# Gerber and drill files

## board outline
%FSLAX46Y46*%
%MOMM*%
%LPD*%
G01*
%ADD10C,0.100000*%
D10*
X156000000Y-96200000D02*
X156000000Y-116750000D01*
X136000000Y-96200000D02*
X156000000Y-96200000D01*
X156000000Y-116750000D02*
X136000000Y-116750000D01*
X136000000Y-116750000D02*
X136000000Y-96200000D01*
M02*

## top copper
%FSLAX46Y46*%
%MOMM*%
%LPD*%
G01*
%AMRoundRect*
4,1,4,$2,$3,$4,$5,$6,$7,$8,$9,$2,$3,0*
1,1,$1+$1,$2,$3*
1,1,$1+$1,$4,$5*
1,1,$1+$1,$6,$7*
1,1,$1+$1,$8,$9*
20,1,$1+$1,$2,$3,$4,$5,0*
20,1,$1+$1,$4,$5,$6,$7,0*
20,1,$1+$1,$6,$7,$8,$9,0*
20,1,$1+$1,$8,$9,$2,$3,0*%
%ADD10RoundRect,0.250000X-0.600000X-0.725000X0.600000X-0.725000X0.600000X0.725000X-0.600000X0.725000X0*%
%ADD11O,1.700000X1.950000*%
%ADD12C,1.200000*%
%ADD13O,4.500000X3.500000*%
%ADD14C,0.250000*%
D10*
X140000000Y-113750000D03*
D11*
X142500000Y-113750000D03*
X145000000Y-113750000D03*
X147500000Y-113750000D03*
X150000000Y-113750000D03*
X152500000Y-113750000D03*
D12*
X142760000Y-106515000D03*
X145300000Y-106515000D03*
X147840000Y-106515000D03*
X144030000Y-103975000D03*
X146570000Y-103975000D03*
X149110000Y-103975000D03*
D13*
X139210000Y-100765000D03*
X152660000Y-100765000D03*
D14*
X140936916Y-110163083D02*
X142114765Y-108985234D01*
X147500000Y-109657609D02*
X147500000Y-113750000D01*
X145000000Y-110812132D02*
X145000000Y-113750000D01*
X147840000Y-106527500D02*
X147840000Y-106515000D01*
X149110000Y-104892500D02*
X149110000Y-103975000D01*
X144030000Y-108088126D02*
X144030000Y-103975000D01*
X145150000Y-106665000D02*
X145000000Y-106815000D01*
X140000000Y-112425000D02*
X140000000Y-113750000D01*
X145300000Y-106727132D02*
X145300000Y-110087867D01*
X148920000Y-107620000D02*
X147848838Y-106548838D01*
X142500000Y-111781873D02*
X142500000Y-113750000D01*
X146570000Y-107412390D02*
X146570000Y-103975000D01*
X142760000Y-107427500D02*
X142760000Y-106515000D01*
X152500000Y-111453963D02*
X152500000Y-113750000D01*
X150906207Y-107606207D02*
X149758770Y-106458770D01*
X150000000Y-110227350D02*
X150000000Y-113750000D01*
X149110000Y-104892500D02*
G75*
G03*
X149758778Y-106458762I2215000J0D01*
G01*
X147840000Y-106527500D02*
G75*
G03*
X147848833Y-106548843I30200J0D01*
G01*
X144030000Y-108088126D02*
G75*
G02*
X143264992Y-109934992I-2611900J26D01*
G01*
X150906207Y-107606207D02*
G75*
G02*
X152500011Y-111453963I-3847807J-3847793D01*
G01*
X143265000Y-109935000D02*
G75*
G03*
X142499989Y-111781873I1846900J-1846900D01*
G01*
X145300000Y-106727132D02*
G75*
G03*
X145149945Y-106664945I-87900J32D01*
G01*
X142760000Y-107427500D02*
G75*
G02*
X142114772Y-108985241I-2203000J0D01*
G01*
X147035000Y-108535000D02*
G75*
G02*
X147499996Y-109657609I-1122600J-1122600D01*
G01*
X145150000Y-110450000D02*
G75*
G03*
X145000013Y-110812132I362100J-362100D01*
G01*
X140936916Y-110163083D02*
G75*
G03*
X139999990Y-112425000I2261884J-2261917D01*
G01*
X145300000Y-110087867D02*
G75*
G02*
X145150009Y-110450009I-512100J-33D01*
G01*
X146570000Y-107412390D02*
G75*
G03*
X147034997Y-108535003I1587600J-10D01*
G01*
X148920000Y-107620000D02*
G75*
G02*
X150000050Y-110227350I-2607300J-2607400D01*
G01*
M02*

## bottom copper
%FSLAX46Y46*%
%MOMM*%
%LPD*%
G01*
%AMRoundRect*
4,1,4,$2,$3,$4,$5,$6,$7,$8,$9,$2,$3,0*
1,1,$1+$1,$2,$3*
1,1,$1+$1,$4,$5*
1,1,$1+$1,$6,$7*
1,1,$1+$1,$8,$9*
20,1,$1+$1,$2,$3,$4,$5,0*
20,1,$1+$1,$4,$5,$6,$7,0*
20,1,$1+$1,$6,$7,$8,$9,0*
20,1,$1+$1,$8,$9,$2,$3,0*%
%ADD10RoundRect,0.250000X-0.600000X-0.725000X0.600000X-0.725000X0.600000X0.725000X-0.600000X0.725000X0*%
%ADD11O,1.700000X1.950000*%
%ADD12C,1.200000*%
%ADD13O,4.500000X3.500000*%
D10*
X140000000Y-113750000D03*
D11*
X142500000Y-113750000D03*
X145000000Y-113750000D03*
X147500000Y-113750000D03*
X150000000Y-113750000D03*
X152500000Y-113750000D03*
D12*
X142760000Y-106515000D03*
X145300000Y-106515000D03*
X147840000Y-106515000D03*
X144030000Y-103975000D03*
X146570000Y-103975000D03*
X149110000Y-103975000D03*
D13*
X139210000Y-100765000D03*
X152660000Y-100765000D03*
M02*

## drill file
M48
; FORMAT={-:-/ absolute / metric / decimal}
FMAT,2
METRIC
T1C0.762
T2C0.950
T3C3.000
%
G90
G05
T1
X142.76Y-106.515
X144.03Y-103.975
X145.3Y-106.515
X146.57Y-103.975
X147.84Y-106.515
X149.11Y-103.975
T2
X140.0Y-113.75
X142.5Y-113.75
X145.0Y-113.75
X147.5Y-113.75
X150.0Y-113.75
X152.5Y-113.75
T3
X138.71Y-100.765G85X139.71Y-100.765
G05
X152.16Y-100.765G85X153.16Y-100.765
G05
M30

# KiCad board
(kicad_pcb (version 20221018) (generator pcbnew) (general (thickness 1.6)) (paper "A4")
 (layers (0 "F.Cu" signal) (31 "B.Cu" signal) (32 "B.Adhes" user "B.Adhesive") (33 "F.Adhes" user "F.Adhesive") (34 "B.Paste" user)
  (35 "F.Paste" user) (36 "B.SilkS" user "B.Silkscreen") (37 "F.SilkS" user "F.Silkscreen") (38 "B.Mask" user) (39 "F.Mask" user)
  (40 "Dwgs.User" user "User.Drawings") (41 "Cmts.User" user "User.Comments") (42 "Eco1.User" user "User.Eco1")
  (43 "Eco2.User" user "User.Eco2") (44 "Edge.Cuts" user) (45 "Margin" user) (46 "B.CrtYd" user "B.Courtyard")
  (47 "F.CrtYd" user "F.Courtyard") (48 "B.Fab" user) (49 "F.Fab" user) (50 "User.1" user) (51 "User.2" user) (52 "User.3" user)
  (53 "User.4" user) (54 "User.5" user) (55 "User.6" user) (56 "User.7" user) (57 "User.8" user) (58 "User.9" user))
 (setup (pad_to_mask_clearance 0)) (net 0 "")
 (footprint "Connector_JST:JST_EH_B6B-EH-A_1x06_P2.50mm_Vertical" (layer "F.Cu") (at 140 113.75)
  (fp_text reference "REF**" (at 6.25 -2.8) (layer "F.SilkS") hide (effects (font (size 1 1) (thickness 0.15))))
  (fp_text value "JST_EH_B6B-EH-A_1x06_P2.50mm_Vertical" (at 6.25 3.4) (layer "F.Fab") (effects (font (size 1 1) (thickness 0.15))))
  (pad "1" thru_hole roundrect (at 0 0) (size 1.7 1.95) (drill 0.95) (layers "*.Cu" "*.Mask") (roundrect_rratio 0.1470588235))
  (pad "2" thru_hole oval (at 2.5 0) (size 1.7 1.95) (drill 0.95) (layers "*.Cu" "*.Mask"))
  (pad "3" thru_hole oval (at 5 0) (size 1.7 1.95) (drill 0.95) (layers "*.Cu" "*.Mask"))
  (pad "4" thru_hole oval (at 7.5 0) (size 1.7 1.95) (drill 0.95) (layers "*.Cu" "*.Mask"))
  (pad "5" thru_hole oval (at 10 0) (size 1.7 1.95) (drill 0.95) (layers "*.Cu" "*.Mask"))
  (pad "6" thru_hole oval (at 12.5 0) (size 1.7 1.95) (drill 0.95) (layers "*.Cu" "*.Mask")))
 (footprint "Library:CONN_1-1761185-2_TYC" (layer "F.Cu") (at 142.76 106.515)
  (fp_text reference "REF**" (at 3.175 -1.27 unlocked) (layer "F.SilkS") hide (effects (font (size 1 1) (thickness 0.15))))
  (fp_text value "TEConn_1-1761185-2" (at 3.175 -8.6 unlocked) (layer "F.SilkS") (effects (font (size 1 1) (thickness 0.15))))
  (pad "1" thru_hole circle (at 0 0) (size 1.2 1.2) (drill 0.762) (layers "*.Cu" "*.Mask"))
  (pad "3" thru_hole circle (at 2.54 0) (size 1.2 1.2) (drill 0.762) (layers "*.Cu" "*.Mask"))
  (pad "5" thru_hole circle (at 5.08 0) (size 1.2 1.2) (drill 0.762) (layers "*.Cu" "*.Mask"))
  (pad "8" thru_hole circle (at 1.27 -2.54) (size 1.2 1.2) (drill 0.762) (layers "*.Cu" "*.Mask"))
  (pad "10" thru_hole circle (at 3.81 -2.54) (size 1.2 1.2) (drill 0.762) (layers "*.Cu" "*.Mask"))
  (pad "12" thru_hole circle (at 6.35 -2.54) (size 1.2 1.2) (drill 0.762) (layers "*.Cu" "*.Mask"))
  (pad "13" thru_hole oval (at -3.55 -5.75) (size 4.5 3.5) (drill oval 4 3) (layers "*.Cu" "*.Mask"))
  (pad "14" thru_hole oval (at 9.9 -5.75) (size 4.5 3.5) (drill oval 4 3) (layers "*.Cu" "*.Mask")))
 (gr_line (start 156 96.2) (end 156 116.75) (stroke (width 0.1) (type default)) (layer "Edge.Cuts"))
 (gr_line (start 136 96.2) (end 156 96.2) (stroke (width 0.1) (type default)) (layer "Edge.Cuts"))
 (gr_line (start 156 116.75) (end 136 116.75) (stroke (width 0.1) (type default)) (layer "Edge.Cuts"))
 (gr_line (start 136 116.75) (end 136 96.2) (stroke (width 0.1) (type default)) (layer "Edge.Cuts"))
 (segment (start 140.936916 110.163083) (end 142.114765 108.985234) (width 0.25) (layer "F.Cu") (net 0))
 (segment (start 147.5 109.657609) (end 147.5 113.75) (width 0.25) (layer "F.Cu") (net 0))
 (segment (start 145 110.812132) (end 145 113.75) (width 0.25) (layer "F.Cu") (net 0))
 (segment (start 147.84 106.5275) (end 147.84 106.515) (width 0.25) (layer "F.Cu") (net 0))
 (segment (start 149.11 104.8925) (end 149.11 103.975) (width 0.25) (layer "F.Cu") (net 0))
 (segment (start 144.03 108.088126) (end 144.03 103.975) (width 0.25) (layer "F.Cu") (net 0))
 (segment (start 145.15 106.665) (end 145 106.815) (width 0.25) (layer "F.Cu") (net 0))
 (segment (start 140 112.425) (end 140 113.75) (width 0.25) (layer "F.Cu") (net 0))
 (segment (start 145.3 106.727132) (end 145.3 110.087867) (width 0.25) (layer "F.Cu") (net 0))
 (segment (start 148.92 107.62) (end 147.848838 106.548838) (width 0.25) (layer "F.Cu") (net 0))
 (segment (start 142.5 111.781873) (end 142.5 113.75) (width 0.25) (layer "F.Cu") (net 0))
 (segment (start 146.57 107.41239) (end 146.57 103.975) (width 0.25) (layer "F.Cu") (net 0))
 (segment (start 142.76 107.4275) (end 142.76 106.515) (width 0.25) (layer "F.Cu") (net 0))
 (segment (start 152.5 111.453963) (end 152.5 113.75) (width 0.25) (layer "F.Cu") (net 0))
 (segment (start 150.906207 107.606207) (end 149.75877 106.45877) (width 0.25) (layer "F.Cu") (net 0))
 (segment (start 150 110.22735) (end 150 113.75) (width 0.25) (layer "F.Cu") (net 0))
 (arc (start 149.11 104.8925) (mid 149.278609 105.740159) (end 149.75877 106.45877) (width 0.25) (layer "F.Cu") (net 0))
 (arc (start 147.84 106.5275) (mid 147.842296 106.539048) (end 147.848838 106.548838) (width 0.25) (layer "F.Cu") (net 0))
 (arc (start 144.03 108.088126) (mid 143.831182 109.087647) (end 143.265 109.935) (width 0.25) (layer "F.Cu") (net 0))
 (arc (start 150.906207 107.606207) (mid 152.085786 109.371572) (end 152.5 111.453963) (width 0.25) (layer "F.Cu") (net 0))
 (arc (start 143.265 109.935) (mid 142.698817 110.782352) (end 142.5 111.781873) (width 0.25) (layer "F.Cu") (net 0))
 (arc (start 145.3 106.727132) (mid 145.245757 106.645952) (end 145.15 106.665) (width 0.25) (layer "F.Cu") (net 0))
 (arc (start 142.76 107.4275) (mid 142.592308 108.270539) (end 142.114765 108.985234) (width 0.25) (layer "F.Cu") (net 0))
 (arc (start 147.035 108.535) (mid 147.37915 109.050057) (end 147.5 109.657609) (width 0.25) (layer "F.Cu") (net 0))
 (arc (start 145.15 110.45) (mid 145.038983 110.616147) (end 145 110.812132) (width 0.25) (layer "F.Cu") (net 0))
 (arc (start 140.936916 110.163083) (mid 140.243496 111.200859) (end 140 112.425) (width 0.25) (layer "F.Cu") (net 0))
 (arc (start 145.3 110.087867) (mid 145.261016 110.283852) (end 145.15 110.45) (width 0.25) (layer "F.Cu") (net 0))
 (arc (start 146.57 107.41239) (mid 146.690849 108.019942) (end 147.035 108.535) (width 0.25) (layer "F.Cu") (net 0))
 (arc (start 148.92 107.62) (mid 149.719317 108.816262) (end 150 110.22735) (width 0.25) (layer "F.Cu") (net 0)))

